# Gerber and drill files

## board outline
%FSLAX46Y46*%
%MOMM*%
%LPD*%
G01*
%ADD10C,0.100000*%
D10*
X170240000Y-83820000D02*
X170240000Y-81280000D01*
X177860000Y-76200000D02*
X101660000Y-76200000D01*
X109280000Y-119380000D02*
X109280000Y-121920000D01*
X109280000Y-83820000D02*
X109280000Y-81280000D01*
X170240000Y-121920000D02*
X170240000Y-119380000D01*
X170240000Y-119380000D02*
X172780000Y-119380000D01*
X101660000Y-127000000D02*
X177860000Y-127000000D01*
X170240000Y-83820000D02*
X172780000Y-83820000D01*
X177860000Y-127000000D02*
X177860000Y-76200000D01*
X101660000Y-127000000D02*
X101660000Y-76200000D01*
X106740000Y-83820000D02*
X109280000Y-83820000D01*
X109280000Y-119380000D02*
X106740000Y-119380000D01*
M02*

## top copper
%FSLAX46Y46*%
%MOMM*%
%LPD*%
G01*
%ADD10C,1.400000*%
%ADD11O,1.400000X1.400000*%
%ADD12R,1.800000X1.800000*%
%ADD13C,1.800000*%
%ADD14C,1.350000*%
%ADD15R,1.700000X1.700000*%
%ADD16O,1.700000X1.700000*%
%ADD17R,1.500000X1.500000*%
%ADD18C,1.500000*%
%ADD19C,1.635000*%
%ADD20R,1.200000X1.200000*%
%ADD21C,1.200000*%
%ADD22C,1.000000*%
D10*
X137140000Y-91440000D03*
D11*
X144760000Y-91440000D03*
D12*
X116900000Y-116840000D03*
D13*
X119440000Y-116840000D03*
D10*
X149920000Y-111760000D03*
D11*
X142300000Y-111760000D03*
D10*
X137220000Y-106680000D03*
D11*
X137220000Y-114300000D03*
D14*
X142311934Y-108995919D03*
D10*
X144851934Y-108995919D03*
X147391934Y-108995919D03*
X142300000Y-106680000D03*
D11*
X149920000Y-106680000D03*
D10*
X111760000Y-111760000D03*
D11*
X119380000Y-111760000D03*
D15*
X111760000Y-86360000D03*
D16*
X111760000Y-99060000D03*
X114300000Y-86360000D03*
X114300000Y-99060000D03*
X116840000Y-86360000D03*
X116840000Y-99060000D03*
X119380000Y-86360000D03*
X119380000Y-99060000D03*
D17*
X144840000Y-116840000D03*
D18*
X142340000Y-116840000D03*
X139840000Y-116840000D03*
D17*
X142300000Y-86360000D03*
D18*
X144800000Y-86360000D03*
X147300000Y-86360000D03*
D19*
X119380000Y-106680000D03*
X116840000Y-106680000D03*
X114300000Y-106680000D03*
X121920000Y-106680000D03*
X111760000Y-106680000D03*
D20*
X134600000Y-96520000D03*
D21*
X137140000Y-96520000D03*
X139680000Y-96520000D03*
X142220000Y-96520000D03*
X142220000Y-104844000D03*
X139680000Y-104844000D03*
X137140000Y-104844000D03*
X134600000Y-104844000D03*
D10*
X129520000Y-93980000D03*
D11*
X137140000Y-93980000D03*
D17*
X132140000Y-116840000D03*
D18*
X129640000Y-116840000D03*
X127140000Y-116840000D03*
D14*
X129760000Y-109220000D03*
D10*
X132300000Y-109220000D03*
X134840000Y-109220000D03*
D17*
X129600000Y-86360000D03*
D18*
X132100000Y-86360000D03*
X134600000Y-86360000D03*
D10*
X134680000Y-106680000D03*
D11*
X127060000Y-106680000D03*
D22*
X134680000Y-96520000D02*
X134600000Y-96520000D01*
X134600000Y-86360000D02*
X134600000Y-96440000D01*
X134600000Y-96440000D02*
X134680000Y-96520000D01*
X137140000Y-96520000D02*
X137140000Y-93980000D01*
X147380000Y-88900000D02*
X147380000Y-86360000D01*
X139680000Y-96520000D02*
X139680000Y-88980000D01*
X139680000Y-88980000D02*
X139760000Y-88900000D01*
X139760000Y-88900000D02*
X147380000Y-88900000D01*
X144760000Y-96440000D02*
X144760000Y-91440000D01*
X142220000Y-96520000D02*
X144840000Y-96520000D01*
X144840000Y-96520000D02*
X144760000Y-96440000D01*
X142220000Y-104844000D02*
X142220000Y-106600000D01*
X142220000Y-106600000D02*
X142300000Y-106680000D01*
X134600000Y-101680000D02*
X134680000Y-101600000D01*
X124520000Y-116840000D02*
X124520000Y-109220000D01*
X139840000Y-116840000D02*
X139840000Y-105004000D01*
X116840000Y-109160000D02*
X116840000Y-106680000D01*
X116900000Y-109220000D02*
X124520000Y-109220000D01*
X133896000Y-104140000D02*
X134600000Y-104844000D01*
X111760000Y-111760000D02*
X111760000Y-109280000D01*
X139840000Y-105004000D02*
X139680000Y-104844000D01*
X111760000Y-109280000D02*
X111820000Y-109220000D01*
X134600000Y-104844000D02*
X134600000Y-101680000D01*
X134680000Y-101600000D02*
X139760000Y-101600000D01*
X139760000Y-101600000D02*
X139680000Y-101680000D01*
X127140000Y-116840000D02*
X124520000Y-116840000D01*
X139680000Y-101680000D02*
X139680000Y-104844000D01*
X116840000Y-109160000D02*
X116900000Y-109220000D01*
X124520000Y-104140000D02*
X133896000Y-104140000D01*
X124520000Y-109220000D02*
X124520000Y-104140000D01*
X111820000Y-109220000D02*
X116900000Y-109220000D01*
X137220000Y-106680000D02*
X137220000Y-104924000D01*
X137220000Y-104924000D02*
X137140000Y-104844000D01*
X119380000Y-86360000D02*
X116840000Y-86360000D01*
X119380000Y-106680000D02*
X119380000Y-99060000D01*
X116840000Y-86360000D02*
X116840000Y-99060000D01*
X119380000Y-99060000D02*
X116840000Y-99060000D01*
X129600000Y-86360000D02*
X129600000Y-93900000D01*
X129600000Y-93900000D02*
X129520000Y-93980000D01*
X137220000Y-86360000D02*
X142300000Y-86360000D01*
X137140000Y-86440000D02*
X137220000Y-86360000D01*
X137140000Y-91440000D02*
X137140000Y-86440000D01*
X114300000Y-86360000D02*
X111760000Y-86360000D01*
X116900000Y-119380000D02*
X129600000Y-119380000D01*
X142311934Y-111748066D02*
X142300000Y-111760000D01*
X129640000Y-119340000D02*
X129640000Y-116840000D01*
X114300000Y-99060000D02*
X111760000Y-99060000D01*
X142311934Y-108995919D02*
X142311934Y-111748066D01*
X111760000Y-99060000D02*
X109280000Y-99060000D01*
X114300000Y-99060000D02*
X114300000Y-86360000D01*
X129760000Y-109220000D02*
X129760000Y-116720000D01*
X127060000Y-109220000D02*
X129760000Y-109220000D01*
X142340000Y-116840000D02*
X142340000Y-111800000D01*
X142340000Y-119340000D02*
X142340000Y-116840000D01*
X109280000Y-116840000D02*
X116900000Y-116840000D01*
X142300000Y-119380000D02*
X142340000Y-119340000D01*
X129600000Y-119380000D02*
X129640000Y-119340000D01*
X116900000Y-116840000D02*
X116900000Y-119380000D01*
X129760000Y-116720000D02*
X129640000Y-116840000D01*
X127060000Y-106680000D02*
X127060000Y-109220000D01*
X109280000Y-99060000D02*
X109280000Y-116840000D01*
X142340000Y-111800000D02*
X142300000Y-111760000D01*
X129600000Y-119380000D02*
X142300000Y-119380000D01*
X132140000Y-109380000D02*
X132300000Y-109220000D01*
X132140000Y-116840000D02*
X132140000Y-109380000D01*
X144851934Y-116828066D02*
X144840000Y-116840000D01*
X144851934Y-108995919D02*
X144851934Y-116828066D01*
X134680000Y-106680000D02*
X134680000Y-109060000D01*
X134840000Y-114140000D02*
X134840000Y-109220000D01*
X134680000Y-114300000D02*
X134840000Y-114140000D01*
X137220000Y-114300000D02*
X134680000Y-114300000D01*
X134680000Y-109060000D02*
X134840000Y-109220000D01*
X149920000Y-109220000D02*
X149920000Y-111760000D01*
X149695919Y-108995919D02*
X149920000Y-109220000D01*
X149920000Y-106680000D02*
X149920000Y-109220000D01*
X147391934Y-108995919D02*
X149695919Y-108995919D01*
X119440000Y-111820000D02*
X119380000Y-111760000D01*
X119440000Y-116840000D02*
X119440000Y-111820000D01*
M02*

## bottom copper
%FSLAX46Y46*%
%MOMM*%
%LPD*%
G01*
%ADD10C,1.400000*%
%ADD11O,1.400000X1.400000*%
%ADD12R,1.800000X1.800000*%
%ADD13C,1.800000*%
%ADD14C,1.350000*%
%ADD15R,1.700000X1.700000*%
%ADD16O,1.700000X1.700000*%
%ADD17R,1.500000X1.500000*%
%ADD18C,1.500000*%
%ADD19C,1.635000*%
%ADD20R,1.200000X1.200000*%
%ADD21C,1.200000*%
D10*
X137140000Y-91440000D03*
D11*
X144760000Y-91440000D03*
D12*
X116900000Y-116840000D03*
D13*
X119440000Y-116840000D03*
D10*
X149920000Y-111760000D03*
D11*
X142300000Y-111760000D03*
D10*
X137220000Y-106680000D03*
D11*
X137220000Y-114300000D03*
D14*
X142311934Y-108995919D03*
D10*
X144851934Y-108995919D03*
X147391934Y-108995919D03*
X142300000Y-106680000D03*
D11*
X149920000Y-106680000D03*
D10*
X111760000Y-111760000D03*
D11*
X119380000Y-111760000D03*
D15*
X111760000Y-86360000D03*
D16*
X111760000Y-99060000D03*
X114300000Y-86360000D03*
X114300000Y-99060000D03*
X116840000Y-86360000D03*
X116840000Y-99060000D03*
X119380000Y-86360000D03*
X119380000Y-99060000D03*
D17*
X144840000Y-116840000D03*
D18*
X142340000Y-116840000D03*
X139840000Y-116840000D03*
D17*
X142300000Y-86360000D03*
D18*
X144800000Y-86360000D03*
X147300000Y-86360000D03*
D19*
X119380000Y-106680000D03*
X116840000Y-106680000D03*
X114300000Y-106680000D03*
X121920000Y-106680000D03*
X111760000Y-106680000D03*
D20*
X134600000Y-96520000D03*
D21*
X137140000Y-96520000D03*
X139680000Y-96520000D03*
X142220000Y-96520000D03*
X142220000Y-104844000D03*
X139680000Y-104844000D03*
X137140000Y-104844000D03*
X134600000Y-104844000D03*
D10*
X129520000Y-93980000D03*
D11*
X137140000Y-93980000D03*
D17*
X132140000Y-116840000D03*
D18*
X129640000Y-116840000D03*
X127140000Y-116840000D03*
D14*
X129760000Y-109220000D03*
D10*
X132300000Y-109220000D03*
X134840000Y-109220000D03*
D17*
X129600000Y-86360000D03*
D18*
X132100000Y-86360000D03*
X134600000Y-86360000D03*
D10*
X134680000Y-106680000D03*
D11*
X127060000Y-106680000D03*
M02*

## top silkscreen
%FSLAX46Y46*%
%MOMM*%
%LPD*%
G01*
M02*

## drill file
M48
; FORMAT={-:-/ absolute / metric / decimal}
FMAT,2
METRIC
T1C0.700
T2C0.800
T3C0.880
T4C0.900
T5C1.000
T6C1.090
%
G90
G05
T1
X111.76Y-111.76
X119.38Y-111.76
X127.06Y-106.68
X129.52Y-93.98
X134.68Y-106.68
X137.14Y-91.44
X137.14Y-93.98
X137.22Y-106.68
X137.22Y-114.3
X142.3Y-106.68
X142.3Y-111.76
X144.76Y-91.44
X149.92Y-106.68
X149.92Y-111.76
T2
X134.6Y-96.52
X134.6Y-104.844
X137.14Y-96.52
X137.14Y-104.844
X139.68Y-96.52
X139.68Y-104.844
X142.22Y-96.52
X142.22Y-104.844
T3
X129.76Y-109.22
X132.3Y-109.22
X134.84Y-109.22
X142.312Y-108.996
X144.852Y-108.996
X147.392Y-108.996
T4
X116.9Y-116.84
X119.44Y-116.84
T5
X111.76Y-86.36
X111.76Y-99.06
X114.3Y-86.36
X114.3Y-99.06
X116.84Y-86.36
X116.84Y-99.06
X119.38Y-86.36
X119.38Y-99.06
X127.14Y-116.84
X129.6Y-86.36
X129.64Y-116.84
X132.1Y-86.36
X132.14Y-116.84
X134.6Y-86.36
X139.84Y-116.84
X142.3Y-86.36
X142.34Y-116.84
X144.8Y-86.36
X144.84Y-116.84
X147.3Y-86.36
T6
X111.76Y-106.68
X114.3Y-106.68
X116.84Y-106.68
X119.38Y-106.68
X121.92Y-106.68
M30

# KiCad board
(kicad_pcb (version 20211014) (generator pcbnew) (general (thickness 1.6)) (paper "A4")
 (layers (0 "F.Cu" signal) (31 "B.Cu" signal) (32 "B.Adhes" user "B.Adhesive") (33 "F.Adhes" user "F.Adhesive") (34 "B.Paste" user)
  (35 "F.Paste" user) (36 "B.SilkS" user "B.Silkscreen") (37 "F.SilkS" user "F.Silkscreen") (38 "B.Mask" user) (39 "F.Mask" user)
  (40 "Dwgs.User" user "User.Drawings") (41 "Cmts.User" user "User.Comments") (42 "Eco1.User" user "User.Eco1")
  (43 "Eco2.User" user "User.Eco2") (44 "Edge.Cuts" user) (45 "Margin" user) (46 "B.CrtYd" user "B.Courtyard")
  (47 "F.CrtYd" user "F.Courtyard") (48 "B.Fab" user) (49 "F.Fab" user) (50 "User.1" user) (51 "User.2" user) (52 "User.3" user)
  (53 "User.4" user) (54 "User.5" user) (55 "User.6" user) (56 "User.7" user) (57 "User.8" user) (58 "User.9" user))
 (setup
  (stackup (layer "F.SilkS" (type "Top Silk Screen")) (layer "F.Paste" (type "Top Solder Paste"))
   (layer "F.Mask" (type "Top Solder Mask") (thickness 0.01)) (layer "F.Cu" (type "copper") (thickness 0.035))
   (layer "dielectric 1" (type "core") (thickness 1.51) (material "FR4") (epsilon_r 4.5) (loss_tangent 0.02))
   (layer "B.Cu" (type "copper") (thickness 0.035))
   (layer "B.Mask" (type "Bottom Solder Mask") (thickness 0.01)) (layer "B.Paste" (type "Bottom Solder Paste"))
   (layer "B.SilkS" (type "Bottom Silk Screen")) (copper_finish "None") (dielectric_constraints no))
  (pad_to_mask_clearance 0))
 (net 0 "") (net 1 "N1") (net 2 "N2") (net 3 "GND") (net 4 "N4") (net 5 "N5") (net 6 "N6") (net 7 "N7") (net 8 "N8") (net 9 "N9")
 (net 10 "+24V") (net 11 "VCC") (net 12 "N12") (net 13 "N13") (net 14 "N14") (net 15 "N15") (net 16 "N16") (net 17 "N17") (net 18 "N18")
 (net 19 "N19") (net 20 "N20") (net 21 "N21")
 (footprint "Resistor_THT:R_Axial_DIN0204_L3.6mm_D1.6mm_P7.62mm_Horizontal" (layer "B.Cu") (at 137.14 91.44)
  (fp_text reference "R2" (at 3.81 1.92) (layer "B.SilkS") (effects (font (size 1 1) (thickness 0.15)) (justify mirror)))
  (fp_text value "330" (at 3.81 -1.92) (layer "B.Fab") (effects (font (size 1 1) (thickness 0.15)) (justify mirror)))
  (pad "1" thru_hole circle (at 0 0) (size 1.4 1.4) (drill 0.7) (layers *.Cu *.Mask) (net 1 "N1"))
  (pad "2" thru_hole oval (at 7.62 0) (size 1.4 1.4) (drill 0.7) (layers *.Cu *.Mask) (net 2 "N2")))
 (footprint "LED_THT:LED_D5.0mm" (layer "B.Cu") (at 116.9 116.84)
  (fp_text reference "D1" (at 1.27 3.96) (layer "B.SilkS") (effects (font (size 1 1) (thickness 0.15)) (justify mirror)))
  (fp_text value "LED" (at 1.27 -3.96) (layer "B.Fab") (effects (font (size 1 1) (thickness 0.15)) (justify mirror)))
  (pad "1" thru_hole rect (at 0 0) (size 1.8 1.8) (drill 0.9) (layers *.Cu *.Mask) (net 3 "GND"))
  (pad "2" thru_hole circle (at 2.54 0) (size 1.8 1.8) (drill 0.9) (layers *.Cu *.Mask) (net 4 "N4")))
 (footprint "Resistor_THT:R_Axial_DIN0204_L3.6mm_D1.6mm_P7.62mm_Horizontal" (layer "B.Cu") (at 149.92 111.76 180)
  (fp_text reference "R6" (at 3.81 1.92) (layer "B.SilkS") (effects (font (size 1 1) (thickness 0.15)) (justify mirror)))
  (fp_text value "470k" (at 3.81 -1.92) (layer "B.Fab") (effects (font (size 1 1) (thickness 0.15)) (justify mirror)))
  (pad "1" thru_hole circle (at 0 0 180) (size 1.4 1.4) (drill 0.7) (layers *.Cu *.Mask) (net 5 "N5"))
  (pad "2" thru_hole oval (at 7.62 0 180) (size 1.4 1.4) (drill 0.7) (layers *.Cu *.Mask) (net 3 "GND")))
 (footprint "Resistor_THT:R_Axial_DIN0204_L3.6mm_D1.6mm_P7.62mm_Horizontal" (layer "B.Cu") (at 137.22 106.68 -90)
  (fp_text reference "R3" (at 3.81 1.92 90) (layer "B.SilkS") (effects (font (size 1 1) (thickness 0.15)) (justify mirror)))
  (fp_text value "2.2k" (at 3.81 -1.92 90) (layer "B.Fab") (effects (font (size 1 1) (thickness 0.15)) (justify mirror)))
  (pad "1" thru_hole circle (at 0 0 270) (size 1.4 1.4) (drill 0.7) (layers *.Cu *.Mask) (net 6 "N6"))
  (pad "2" thru_hole oval (at 7.62 0 270) (size 1.4 1.4) (drill 0.7) (layers *.Cu *.Mask) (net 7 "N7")))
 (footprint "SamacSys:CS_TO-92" (layer "B.Cu") (at 144.851934 111.535919)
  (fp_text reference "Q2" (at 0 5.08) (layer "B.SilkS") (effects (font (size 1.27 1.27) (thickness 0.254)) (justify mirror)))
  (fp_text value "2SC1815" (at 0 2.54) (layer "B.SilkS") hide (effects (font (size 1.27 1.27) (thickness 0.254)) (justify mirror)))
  (pad "1" thru_hole circle (at -2.54 -2.54) (size 1.35 1.35) (drill 0.88) (layers *.Cu *.Mask) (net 3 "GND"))
  (pad "2" thru_hole circle (at 0 -2.54) (size 1.4 1.4) (drill 0.88) (layers *.Cu *.Mask) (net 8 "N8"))
  (pad "3" thru_hole circle (at 2.54 -2.54) (size 1.4 1.4) (drill 0.88) (layers *.Cu *.Mask) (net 5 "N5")))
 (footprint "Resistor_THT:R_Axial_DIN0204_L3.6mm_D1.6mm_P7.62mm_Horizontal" (layer "B.Cu") (at 142.3 106.68)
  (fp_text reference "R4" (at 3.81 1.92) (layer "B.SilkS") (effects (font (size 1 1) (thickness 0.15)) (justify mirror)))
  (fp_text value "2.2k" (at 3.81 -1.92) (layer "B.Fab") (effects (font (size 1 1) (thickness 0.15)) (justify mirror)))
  (pad "1" thru_hole circle (at 0 0) (size 1.4 1.4) (drill 0.7) (layers *.Cu *.Mask) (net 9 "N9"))
  (pad "2" thru_hole oval (at 7.62 0) (size 1.4 1.4) (drill 0.7) (layers *.Cu *.Mask) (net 5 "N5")))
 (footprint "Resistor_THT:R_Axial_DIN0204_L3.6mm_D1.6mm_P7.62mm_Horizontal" (layer "B.Cu") (at 111.76 111.76)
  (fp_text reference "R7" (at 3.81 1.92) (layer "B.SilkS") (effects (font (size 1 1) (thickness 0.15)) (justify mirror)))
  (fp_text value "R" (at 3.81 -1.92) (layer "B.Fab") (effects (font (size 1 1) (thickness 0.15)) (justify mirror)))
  (pad "1" thru_hole circle (at 0 0) (size 1.4 1.4) (drill 0.7) (layers *.Cu *.Mask) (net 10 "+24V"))
  (pad "2" thru_hole oval (at 7.62 0) (size 1.4 1.4) (drill 0.7) (layers *.Cu *.Mask) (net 4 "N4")))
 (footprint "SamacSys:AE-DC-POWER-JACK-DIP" (layer "B.Cu") (at 111.76 86.36 -90)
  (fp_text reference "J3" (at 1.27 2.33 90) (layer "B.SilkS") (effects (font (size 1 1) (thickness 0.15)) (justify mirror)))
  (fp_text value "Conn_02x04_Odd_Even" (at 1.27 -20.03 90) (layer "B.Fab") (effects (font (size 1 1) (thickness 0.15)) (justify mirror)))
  (pad "1" thru_hole rect (at 0 0 270) (size 1.7 1.7) (drill 1) (layers *.Cu *.Mask) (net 3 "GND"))
  (pad "2" thru_hole oval (at 12.7 0 270) (size 1.7 1.7) (drill 1) (layers *.Cu *.Mask) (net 3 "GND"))
  (pad "3" thru_hole oval (at 0 -2.54 270) (size 1.7 1.7) (drill 1) (layers *.Cu *.Mask) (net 3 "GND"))
  (pad "4" thru_hole oval (at 12.7 -2.54 270) (size 1.7 1.7) (drill 1) (layers *.Cu *.Mask) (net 3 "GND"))
  (pad "5" thru_hole oval (at 0 -5.08 270) (size 1.7 1.7) (drill 1) (layers *.Cu *.Mask) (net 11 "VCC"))
  (pad "6" thru_hole oval (at 12.7 -5.08 270) (size 1.7 1.7) (drill 1) (layers *.Cu *.Mask) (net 11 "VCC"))
  (pad "7" thru_hole oval (at 0 -7.62 270) (size 1.7 1.7) (drill 1) (layers *.Cu *.Mask) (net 11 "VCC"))
  (pad "8" thru_hole oval (at 12.7 -7.62 270) (size 1.7 1.7) (drill 1) (layers *.Cu *.Mask) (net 11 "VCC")))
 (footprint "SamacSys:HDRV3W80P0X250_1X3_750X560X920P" (layer "B.Cu") (at 144.84 116.84 180)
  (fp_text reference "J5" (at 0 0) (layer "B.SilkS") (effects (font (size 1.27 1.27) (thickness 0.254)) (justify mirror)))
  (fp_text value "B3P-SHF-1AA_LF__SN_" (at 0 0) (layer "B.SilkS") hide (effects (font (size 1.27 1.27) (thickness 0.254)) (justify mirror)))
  (pad "1" thru_hole rect locked (at 0 0 180) (size 1.5 1.5) (drill 1) (layers *.Cu *.Mask) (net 8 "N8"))
  (pad "2" thru_hole circle locked (at 2.5 0 180) (size 1.5 1.5) (drill 1) (layers *.Cu *.Mask) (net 3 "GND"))
  (pad "3" thru_hole circle locked (at 5 0 180) (size 1.5 1.5) (drill 1) (layers *.Cu *.Mask) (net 10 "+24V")))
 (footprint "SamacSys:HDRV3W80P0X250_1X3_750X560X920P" (layer "B.Cu") (at 142.3 86.36)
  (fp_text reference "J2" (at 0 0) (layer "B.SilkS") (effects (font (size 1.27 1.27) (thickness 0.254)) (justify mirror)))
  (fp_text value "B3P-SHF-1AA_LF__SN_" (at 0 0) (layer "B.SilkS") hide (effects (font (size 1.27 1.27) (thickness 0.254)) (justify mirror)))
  (pad "1" thru_hole rect locked (at 0 0) (size 1.5 1.5) (drill 1) (layers *.Cu *.Mask) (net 1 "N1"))
  (pad "2" thru_hole circle locked (at 2.5 0) (size 1.5 1.5) (drill 1) (layers *.Cu *.Mask) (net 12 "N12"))
  (pad "3" thru_hole circle locked (at 5 0) (size 1.5 1.5) (drill 1) (layers *.Cu *.Mask) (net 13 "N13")))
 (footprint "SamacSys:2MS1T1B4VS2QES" (layer "B.Cu") (at 119.38 106.68 90)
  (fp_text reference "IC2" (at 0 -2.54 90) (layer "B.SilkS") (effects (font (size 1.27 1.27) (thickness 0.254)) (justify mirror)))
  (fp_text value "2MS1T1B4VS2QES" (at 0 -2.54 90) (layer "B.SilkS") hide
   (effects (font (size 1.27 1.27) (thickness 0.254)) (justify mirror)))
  (pad "1" thru_hole circle locked (at 0 0 90) (size 1.635 1.635) (drill 1.09) (layers *.Cu *.Mask) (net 11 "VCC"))
  (pad "2" thru_hole circle locked (at 0 -2.54 90) (size 1.635 1.635) (drill 1.09) (layers *.Cu *.Mask) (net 10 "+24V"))
  (pad "3" thru_hole circle locked (at 0 -5.08 90) (size 1.635 1.635) (drill 1.09) (layers *.Cu *.Mask) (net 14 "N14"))
  (pad "MH1" thru_hole circle locked (at 0 2.54 90) (size 1.635 1.635) (drill 1.09) (layers *.Cu *.Mask) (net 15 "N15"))
  (pad "MH2" thru_hole circle locked (at 0 -7.62 90) (size 1.635 1.635) (drill 1.09) (layers *.Cu *.Mask) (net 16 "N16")))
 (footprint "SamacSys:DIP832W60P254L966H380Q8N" (layer "B.Cu") (at 138.41 100.682 -90)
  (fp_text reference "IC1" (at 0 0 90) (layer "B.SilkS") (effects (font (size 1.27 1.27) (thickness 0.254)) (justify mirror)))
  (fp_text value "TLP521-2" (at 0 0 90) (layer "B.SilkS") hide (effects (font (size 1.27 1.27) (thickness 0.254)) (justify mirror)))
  (pad "1" thru_hole rect locked (at -4.162 3.81 270) (size 1.2 1.2) (drill 0.8) (layers *.Cu *.Mask) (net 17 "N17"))
  (pad "2" thru_hole circle locked (at -4.162 1.27 270) (size 1.2 1.2) (drill 0.8) (layers *.Cu *.Mask) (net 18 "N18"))
  (pad "3" thru_hole circle locked (at -4.162 -1.27 270) (size 1.2 1.2) (drill 0.8) (layers *.Cu *.Mask) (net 13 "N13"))
  (pad "4" thru_hole circle locked (at -4.162 -3.81 270) (size 1.2 1.2) (drill 0.8) (layers *.Cu *.Mask) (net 2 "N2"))
  (pad "5" thru_hole circle locked (at 4.162 -3.81 270) (size 1.2 1.2) (drill 0.8) (layers *.Cu *.Mask) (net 9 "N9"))
  (pad "6" thru_hole circle locked (at 4.162 -1.27 270) (size 1.2 1.2) (drill 0.8) (layers *.Cu *.Mask) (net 10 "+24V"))
  (pad "7" thru_hole circle locked (at 4.162 1.27 270) (size 1.2 1.2) (drill 0.8) (layers *.Cu *.Mask) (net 6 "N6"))
  (pad "8" thru_hole circle locked (at 4.162 3.81 270) (size 1.2 1.2) (drill 0.8) (layers *.Cu *.Mask) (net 10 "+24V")))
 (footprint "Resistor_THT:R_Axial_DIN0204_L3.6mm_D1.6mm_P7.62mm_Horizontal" (layer "B.Cu") (at 129.52 93.98)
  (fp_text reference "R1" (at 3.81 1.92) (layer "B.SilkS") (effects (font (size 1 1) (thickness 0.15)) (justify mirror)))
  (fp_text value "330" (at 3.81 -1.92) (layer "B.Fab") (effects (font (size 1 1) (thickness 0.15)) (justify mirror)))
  (pad "1" thru_hole circle (at 0 0) (size 1.4 1.4) (drill 0.7) (layers *.Cu *.Mask) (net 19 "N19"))
  (pad "2" thru_hole oval (at 7.62 0) (size 1.4 1.4) (drill 0.7) (layers *.Cu *.Mask) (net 18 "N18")))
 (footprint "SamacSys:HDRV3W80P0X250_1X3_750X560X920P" (layer "B.Cu") (at 132.14 116.84 180)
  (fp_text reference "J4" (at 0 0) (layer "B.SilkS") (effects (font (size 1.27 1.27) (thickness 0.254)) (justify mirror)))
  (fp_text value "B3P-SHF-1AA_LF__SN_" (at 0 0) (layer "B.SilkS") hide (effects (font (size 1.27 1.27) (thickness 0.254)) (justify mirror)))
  (pad "1" thru_hole rect locked (at 0 0 180) (size 1.5 1.5) (drill 1) (layers *.Cu *.Mask) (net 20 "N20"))
  (pad "2" thru_hole circle locked (at 2.5 0 180) (size 1.5 1.5) (drill 1) (layers *.Cu *.Mask) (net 3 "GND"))
  (pad "3" thru_hole circle locked (at 5 0 180) (size 1.5 1.5) (drill 1) (layers *.Cu *.Mask) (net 10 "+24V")))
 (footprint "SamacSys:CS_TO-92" (layer "B.Cu") (at 132.3 111.76)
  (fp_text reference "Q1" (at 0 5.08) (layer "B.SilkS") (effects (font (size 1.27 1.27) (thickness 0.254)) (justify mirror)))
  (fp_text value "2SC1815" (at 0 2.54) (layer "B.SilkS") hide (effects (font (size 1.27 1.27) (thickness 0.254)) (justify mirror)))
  (pad "1" thru_hole circle (at -2.54 -2.54) (size 1.35 1.35) (drill 0.88) (layers *.Cu *.Mask) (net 3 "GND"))
  (pad "2" thru_hole circle (at 0 -2.54) (size 1.4 1.4) (drill 0.88) (layers *.Cu *.Mask) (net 20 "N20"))
  (pad "3" thru_hole circle (at 2.54 -2.54) (size 1.4 1.4) (drill 0.88) (layers *.Cu *.Mask) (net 7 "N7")))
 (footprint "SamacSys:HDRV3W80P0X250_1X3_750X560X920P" (layer "B.Cu") (at 129.6 86.36)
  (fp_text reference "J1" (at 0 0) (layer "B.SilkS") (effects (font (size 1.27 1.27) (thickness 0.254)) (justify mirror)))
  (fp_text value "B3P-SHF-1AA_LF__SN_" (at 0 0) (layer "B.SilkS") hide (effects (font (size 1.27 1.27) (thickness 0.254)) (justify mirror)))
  (pad "1" thru_hole rect locked (at 0 0) (size 1.5 1.5) (drill 1) (layers *.Cu *.Mask) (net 19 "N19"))
  (pad "2" thru_hole circle locked (at 2.5 0) (size 1.5 1.5) (drill 1) (layers *.Cu *.Mask) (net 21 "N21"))
  (pad "3" thru_hole circle locked (at 5 0) (size 1.5 1.5) (drill 1) (layers *.Cu *.Mask) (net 17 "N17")))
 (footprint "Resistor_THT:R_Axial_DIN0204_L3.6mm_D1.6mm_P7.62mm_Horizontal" (layer "B.Cu") (at 134.68 106.68 180)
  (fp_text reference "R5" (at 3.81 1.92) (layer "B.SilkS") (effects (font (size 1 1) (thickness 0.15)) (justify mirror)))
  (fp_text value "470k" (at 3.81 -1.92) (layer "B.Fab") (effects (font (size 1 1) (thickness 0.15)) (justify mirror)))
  (pad "1" thru_hole circle (at 0 0 180) (size 1.4 1.4) (drill 0.7) (layers *.Cu *.Mask) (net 7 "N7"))
  (pad "2" thru_hole oval (at 7.62 0 180) (size 1.4 1.4) (drill 0.7) (layers *.Cu *.Mask) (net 3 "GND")))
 (gr_line (start 170.24 83.82) (end 170.24 81.28) (layer "Edge.Cuts") (width 0.1))
 (gr_line (start 177.86 76.2) (end 101.66 76.2) (layer "Edge.Cuts") (width 0.1))
 (gr_line (start 109.28 119.38) (end 109.28 121.92) (layer "Edge.Cuts") (width 0.1))
 (gr_line (start 109.28 83.82) (end 109.28 81.28) (layer "Edge.Cuts") (width 0.1))
 (gr_line (start 170.24 121.92) (end 170.24 119.38) (layer "Edge.Cuts") (width 0.1))
 (gr_line (start 170.24 119.38) (end 172.78 119.38) (layer "Edge.Cuts") (width 0.1))
 (gr_line (start 101.66 127) (end 177.86 127) (layer "Edge.Cuts") (width 0.1))
 (gr_line (start 170.24 83.82) (end 172.78 83.82) (layer "Edge.Cuts") (width 0.1))
 (gr_line (start 177.86 127) (end 177.86 76.2) (layer "Edge.Cuts") (width 0.1))
 (gr_line (start 101.66 127) (end 101.66 76.2) (layer "Edge.Cuts") (width 0.1))
 (gr_line (start 106.74 83.82) (end 109.28 83.82) (layer "Edge.Cuts") (width 0.1))
 (gr_line (start 109.28 119.38) (end 106.74 119.38) (layer "Edge.Cuts") (width 0.1))
 (segment (start 134.68 96.52) (end 134.6 96.52) (width 1) (layer "F.Cu") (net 17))
 (segment (start 134.6 86.36) (end 134.6 96.44) (width 1) (layer "F.Cu") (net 17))
 (segment (start 134.6 96.44) (end 134.68 96.52) (width 1) (layer "F.Cu") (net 17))
 (segment (start 137.14 96.52) (end 137.14 93.98) (width 1) (layer "F.Cu") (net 18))
 (segment (start 147.38 88.9) (end 147.38 86.36) (width 1) (layer "F.Cu") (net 13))
 (segment (start 139.68 96.52) (end 139.68 88.98) (width 1) (layer "F.Cu") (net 13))
 (segment (start 139.68 88.98) (end 139.76 88.9) (width 1) (layer "F.Cu") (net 13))
 (segment (start 139.76 88.9) (end 147.38 88.9) (width 1) (layer "F.Cu") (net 13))
 (segment (start 144.76 96.44) (end 144.76 91.44) (width 1) (layer "F.Cu") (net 2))
 (segment (start 142.22 96.52) (end 144.84 96.52) (width 1) (layer "F.Cu") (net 2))
 (segment (start 144.84 96.52) (end 144.76 96.44) (width 1) (layer "F.Cu") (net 2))
 (segment (start 142.22 104.844) (end 142.22 106.6) (width 1) (layer "F.Cu") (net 9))
 (segment (start 142.22 106.6) (end 142.3 106.68) (width 1) (layer "F.Cu") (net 9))
 (segment (start 134.6 101.68) (end 134.68 101.6) (width 1) (layer "F.Cu") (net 10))
 (segment (start 124.52 116.84) (end 124.52 109.22) (width 1) (layer "F.Cu") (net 10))
 (segment (start 139.84 116.84) (end 139.84 105.004) (width 1) (layer "F.Cu") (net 10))
 (segment (start 116.84 109.16) (end 116.84 106.68) (width 1) (layer "F.Cu") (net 10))
 (segment (start 116.9 109.22) (end 124.52 109.22) (width 1) (layer "F.Cu") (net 10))
 (segment (start 133.896 104.14) (end 134.6 104.844) (width 1) (layer "F.Cu") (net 10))
 (segment (start 111.76 111.76) (end 111.76 109.28) (width 1) (layer "F.Cu") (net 10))
 (segment (start 139.84 105.004) (end 139.68 104.844) (width 1) (layer "F.Cu") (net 10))
 (segment (start 111.76 109.28) (end 111.82 109.22) (width 1) (layer "F.Cu") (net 10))
 (segment (start 134.6 104.844) (end 134.6 101.68) (width 1) (layer "F.Cu") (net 10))
 (segment (start 134.68 101.6) (end 139.76 101.6) (width 1) (layer "F.Cu") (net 10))
 (segment (start 139.76 101.6) (end 139.68 101.68) (width 1) (layer "F.Cu") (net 10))
 (segment (start 127.14 116.84) (end 124.52 116.84) (width 1) (layer "F.Cu") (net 10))
 (segment (start 139.68 101.68) (end 139.68 104.844) (width 1) (layer "F.Cu") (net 10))
 (segment (start 116.84 109.16) (end 116.9 109.22) (width 1) (layer "F.Cu") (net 10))
 (segment (start 124.52 104.14) (end 133.896 104.14) (width 1) (layer "F.Cu") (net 10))
 (segment (start 124.52 109.22) (end 124.52 104.14) (width 1) (layer "F.Cu") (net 10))
 (segment (start 111.82 109.22) (end 116.9 109.22) (width 1) (layer "F.Cu") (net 10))
 (segment (start 137.22 106.68) (end 137.22 104.924) (width 1) (layer "F.Cu") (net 6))
 (segment (start 137.22 104.924) (end 137.14 104.844) (width 1) (layer "F.Cu") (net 6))
 (segment (start 119.38 86.36) (end 116.84 86.36) (width 1) (layer "F.Cu") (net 11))
 (segment (start 119.38 106.68) (end 119.38 99.06) (width 1) (layer "F.Cu") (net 11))
 (segment (start 116.84 86.36) (end 116.84 99.06) (width 1) (layer "F.Cu") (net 11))
 (segment (start 119.38 99.06) (end 116.84 99.06) (width 1) (layer "F.Cu") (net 11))
 (segment (start 129.6 86.36) (end 129.6 93.9) (width 1) (layer "F.Cu") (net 19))
 (segment (start 129.6 93.9) (end 129.52 93.98) (width 1) (layer "F.Cu") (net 19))
 (segment (start 137.22 86.36) (end 142.3 86.36) (width 1) (layer "F.Cu") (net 1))
 (segment (start 137.14 86.44) (end 137.22 86.36) (width 1) (layer "F.Cu") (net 1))
 (segment (start 137.14 91.44) (end 137.14 86.44) (width 1) (layer "F.Cu") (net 1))
 (segment (start 114.3 86.36) (end 111.76 86.36) (width 1) (layer "F.Cu") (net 3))
 (segment (start 116.9 119.38) (end 129.6 119.38) (width 1) (layer "F.Cu") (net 3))
 (segment (start 142.311934 111.748066) (end 142.3 111.76) (width 1) (layer "F.Cu") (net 3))
 (segment (start 129.64 119.34) (end 129.64 116.84) (width 1) (layer "F.Cu") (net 3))
 (segment (start 114.3 99.06) (end 111.76 99.06) (width 1) (layer "F.Cu") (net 3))
 (segment (start 142.311934 108.995919) (end 142.311934 111.748066) (width 1) (layer "F.Cu") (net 3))
 (segment (start 111.76 99.06) (end 109.28 99.06) (width 1) (layer "F.Cu") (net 3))
 (segment (start 114.3 99.06) (end 114.3 86.36) (width 1) (layer "F.Cu") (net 3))
 (segment (start 129.76 109.22) (end 129.76 116.72) (width 1) (layer "F.Cu") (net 3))
 (segment (start 127.06 109.22) (end 129.76 109.22) (width 1) (layer "F.Cu") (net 3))
 (segment (start 142.34 116.84) (end 142.34 111.8) (width 1) (layer "F.Cu") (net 3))
 (segment (start 142.34 119.34) (end 142.34 116.84) (width 1) (layer "F.Cu") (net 3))
 (segment (start 109.28 116.84) (end 116.9 116.84) (width 1) (layer "F.Cu") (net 3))
 (segment (start 142.3 119.38) (end 142.34 119.34) (width 1) (layer "F.Cu") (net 3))
 (segment (start 129.6 119.38) (end 129.64 119.34) (width 1) (layer "F.Cu") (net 3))
 (segment (start 116.9 116.84) (end 116.9 119.38) (width 1) (layer "F.Cu") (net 3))
 (segment (start 129.76 116.72) (end 129.64 116.84) (width 1) (layer "F.Cu") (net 3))
 (segment (start 127.06 106.68) (end 127.06 109.22) (width 1) (layer "F.Cu") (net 3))
 (segment (start 109.28 99.06) (end 109.28 116.84) (width 1) (layer "F.Cu") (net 3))
 (segment (start 142.34 111.8) (end 142.3 111.76) (width 1) (layer "F.Cu") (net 3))
 (segment (start 129.6 119.38) (end 142.3 119.38) (width 1) (layer "F.Cu") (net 3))
 (segment (start 132.14 109.38) (end 132.3 109.22) (width 1) (layer "F.Cu") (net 20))
 (segment (start 132.14 116.84) (end 132.14 109.38) (width 1) (layer "F.Cu") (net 20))
 (segment (start 144.851934 116.828066) (end 144.84 116.84) (width 1) (layer "F.Cu") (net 8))
 (segment (start 144.851934 108.995919) (end 144.851934 116.828066) (width 1) (layer "F.Cu") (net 8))
 (segment (start 134.68 106.68) (end 134.68 109.06) (width 1) (layer "F.Cu") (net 7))
 (segment (start 134.84 114.14) (end 134.84 109.22) (width 1) (layer "F.Cu") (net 7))
 (segment (start 134.68 114.3) (end 134.84 114.14) (width 1) (layer "F.Cu") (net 7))
 (segment (start 137.22 114.3) (end 134.68 114.3) (width 1) (layer "F.Cu") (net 7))
 (segment (start 134.68 109.06) (end 134.84 109.22) (width 1) (layer "F.Cu") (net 7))
 (segment (start 149.92 109.22) (end 149.92 111.76) (width 1) (layer "F.Cu") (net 5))
 (segment (start 149.695919 108.995919) (end 149.92 109.22) (width 1) (layer "F.Cu") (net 5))
 (segment (start 149.92 106.68) (end 149.92 109.22) (width 1) (layer "F.Cu") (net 5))
 (segment (start 147.391934 108.995919) (end 149.695919 108.995919) (width 1) (layer "F.Cu") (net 5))
 (segment (start 119.44 111.82) (end 119.38 111.76) (width 1) (layer "F.Cu") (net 4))
 (segment (start 119.44 116.84) (end 119.44 111.82) (width 1) (layer "F.Cu") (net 4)))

